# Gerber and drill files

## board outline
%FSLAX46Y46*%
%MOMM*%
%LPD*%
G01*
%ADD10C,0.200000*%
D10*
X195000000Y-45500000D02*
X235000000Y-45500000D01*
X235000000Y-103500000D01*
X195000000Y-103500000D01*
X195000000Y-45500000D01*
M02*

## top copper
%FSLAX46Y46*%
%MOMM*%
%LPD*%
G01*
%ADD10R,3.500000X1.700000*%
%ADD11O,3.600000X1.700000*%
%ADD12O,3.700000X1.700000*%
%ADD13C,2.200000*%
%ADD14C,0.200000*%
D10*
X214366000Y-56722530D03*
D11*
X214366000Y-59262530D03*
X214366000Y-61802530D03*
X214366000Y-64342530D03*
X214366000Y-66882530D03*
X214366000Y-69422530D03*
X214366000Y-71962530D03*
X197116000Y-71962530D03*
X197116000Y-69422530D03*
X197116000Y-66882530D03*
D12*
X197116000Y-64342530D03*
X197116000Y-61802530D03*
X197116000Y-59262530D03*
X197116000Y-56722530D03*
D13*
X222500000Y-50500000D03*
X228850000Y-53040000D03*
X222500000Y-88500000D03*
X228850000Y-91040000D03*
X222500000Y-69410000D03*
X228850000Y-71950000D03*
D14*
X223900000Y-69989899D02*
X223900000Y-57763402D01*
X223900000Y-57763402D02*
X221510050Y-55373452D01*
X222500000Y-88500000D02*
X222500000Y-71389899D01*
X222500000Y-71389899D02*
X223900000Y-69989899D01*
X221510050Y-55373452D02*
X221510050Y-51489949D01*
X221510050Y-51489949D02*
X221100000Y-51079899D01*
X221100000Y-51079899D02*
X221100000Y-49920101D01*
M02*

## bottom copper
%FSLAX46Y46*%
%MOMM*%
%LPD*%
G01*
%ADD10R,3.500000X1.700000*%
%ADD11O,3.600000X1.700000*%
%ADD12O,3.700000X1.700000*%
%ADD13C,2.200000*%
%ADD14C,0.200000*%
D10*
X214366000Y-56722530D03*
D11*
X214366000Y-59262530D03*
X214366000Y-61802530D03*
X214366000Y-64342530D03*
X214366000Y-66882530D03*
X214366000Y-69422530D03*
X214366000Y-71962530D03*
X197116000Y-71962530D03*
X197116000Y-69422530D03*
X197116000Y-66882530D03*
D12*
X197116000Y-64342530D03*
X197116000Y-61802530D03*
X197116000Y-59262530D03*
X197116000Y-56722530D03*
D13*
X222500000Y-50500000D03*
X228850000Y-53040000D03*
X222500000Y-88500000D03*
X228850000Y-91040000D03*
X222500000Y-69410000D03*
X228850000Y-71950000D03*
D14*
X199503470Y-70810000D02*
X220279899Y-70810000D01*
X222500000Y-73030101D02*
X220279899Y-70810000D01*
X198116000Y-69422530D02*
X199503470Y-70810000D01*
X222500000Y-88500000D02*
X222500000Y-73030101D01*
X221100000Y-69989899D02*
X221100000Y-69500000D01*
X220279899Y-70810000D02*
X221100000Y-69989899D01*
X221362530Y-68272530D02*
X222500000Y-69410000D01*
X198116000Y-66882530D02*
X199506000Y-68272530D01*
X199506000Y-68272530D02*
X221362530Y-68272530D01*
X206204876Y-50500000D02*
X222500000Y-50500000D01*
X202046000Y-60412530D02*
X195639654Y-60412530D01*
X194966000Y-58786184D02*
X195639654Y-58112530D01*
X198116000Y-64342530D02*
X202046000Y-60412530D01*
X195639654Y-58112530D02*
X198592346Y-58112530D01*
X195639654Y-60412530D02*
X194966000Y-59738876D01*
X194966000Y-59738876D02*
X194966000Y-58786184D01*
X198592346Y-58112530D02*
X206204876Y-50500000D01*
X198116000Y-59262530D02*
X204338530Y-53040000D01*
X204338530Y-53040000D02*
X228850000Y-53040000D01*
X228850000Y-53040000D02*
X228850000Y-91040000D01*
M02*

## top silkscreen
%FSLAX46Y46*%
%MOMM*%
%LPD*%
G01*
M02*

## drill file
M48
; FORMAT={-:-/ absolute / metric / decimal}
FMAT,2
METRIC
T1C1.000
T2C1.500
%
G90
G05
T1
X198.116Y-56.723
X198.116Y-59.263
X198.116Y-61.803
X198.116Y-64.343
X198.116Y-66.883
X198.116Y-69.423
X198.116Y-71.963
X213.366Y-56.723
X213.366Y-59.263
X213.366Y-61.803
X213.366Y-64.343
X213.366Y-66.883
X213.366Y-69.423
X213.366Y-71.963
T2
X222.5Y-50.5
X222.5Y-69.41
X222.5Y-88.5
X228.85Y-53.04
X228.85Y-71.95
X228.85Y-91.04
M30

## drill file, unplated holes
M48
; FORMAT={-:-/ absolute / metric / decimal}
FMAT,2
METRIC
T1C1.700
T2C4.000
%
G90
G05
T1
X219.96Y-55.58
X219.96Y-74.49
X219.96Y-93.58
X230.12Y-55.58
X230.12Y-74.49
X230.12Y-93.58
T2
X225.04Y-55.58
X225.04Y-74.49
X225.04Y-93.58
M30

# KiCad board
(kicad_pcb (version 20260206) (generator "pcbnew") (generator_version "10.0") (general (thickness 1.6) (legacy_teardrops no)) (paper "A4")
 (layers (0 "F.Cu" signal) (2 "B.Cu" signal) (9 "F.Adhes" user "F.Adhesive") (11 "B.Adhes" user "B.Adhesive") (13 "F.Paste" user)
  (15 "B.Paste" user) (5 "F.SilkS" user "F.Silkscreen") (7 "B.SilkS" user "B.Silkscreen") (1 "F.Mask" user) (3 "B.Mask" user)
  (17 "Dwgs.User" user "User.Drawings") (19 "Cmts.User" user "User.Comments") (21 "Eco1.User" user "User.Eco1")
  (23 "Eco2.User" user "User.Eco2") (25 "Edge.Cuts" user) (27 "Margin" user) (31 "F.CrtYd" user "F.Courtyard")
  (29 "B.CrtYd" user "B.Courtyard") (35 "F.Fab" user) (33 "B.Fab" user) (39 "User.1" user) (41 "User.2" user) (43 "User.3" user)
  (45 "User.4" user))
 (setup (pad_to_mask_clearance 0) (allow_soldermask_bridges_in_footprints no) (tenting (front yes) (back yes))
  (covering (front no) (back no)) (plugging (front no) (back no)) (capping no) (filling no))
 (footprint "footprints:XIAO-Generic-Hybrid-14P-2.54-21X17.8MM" (layer "B.Cu") (at 205.741 64.34253 180)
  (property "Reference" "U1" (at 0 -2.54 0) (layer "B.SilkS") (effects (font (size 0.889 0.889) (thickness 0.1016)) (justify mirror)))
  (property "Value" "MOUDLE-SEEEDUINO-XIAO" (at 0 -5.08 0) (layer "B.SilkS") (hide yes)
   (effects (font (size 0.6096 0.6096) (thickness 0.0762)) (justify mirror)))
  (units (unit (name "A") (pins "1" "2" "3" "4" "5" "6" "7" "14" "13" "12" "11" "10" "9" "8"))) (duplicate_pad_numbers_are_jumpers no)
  (pad "1" thru_hole rect (at -7.625 7.62 180) (size 3.5 1.7) (drill 1 (offset -1 0)) (layers "*.Cu" "*.Mask") (remove_unused_layers no)
   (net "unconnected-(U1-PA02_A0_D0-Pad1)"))
  (pad "2" thru_hole oval (at -7.625 5.08 180) (size 3.6 1.7) (drill 1 (offset -1 0)) (layers "*.Cu" "*.Mask") (remove_unused_layers no)
   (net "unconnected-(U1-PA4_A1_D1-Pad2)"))
  (pad "3" thru_hole oval (at -7.625 2.54 180) (size 3.6 1.7) (drill 1 (offset -1 0)) (layers "*.Cu" "*.Mask") (remove_unused_layers no)
   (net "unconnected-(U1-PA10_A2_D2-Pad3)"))
  (pad "4" thru_hole oval (at -7.625 0 180) (size 3.6 1.7) (drill 1 (offset -1 0)) (layers "*.Cu" "*.Mask") (remove_unused_layers no)
   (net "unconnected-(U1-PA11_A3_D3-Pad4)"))
  (pad "5" thru_hole oval (at -7.625 -2.54 180) (size 3.6 1.7) (drill 1 (offset -1 0)) (layers "*.Cu" "*.Mask") (remove_unused_layers no)
   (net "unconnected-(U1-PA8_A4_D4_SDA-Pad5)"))
  (pad "6" thru_hole oval (at -7.625 -5.08) (size 3.6 1.7) (drill 1 (offset 1 0)) (layers "*.Cu" "*.Mask") (remove_unused_layers no)
   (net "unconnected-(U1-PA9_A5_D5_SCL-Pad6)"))
  (pad "7" thru_hole oval (at -7.625 -7.62 180) (size 3.6 1.7) (drill 1 (offset -1 0)) (layers "*.Cu" "*.Mask") (remove_unused_layers no)
   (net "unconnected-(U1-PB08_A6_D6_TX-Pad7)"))
  (pad "8" thru_hole oval (at 7.625 -7.62 180) (size 3.6 1.7) (drill 1 (offset 1 0)) (layers "*.Cu" "*.Mask") (remove_unused_layers no)
   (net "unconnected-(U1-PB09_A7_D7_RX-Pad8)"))
  (pad "9" thru_hole oval (at 7.625 -5.08 180) (size 3.6 1.7) (drill 1 (offset 1 0)) (layers "*.Cu" "*.Mask") (remove_unused_layers no)
   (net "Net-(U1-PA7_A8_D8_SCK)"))
  (pad "10" thru_hole oval (at 7.625 -2.54 180) (size 3.6 1.7) (drill 1 (offset 1 0)) (layers "*.Cu" "*.Mask") (remove_unused_layers no)
   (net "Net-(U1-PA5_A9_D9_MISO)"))
  (pad "11" thru_hole oval (at 7.625 0 180) (size 3.7 1.7) (drill 1 (offset 1 0)) (layers "*.Cu" "*.Mask") (remove_unused_layers no)
   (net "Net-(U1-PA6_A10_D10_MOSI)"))
  (pad "12" thru_hole oval (at 7.625 2.54 180) (size 3.7 1.7) (drill 1 (offset 1 0)) (layers "*.Cu" "*.Mask") (remove_unused_layers no)
   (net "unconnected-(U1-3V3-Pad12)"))
  (pad "13" thru_hole oval (at 7.625 5.08 180) (size 3.7 1.7) (drill 1 (offset 1 0)) (layers "*.Cu" "*.Mask") (remove_unused_layers no)
   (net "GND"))
  (pad "14" thru_hole oval (at 7.625 7.62 180) (size 3.7 1.7) (drill 1 (offset 1 0)) (layers "*.Cu" "*.Mask") (remove_unused_layers no)
   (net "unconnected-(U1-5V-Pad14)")))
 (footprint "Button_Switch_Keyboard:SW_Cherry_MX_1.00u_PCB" (layer "B.Cu") (at 222.5 50.5 180)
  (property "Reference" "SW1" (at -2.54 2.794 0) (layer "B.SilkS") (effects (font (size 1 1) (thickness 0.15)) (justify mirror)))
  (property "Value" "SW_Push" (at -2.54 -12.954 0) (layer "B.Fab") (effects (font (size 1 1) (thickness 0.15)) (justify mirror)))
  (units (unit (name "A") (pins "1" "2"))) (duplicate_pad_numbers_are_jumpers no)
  (pad "" np_thru_hole circle (at -7.62 -5.08 180) (size 1.7 1.7) (drill 1.7) (layers "*.Cu" "*.Mask"))
  (pad "" np_thru_hole circle (at -2.54 -5.08 180) (size 4 4) (drill 4) (layers "*.Cu" "*.Mask"))
  (pad "" np_thru_hole circle (at 2.54 -5.08 180) (size 1.7 1.7) (drill 1.7) (layers "*.Cu" "*.Mask"))
  (pad "1" thru_hole circle (at 0 0 180) (size 2.2 2.2) (drill 1.5) (layers "*.Cu" "*.Mask") (remove_unused_layers no)
   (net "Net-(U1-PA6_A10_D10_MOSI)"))
  (pad "2" thru_hole circle (at -6.35 -2.54 180) (size 2.2 2.2) (drill 1.5) (layers "*.Cu" "*.Mask") (remove_unused_layers no) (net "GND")))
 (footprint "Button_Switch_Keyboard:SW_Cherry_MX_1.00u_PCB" (layer "B.Cu") (at 222.5 88.5 180)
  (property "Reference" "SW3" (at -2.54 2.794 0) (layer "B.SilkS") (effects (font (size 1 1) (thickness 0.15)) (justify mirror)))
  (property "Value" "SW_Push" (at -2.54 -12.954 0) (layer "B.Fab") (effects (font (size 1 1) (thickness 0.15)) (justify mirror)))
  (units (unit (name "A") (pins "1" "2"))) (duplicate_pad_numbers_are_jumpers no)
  (pad "" np_thru_hole circle (at -7.62 -5.08 180) (size 1.7 1.7) (drill 1.7) (layers "*.Cu" "*.Mask"))
  (pad "" np_thru_hole circle (at -2.54 -5.08 180) (size 4 4) (drill 4) (layers "*.Cu" "*.Mask"))
  (pad "" np_thru_hole circle (at 2.54 -5.08 180) (size 1.7 1.7) (drill 1.7) (layers "*.Cu" "*.Mask"))
  (pad "1" thru_hole circle (at 0 0 180) (size 2.2 2.2) (drill 1.5) (layers "*.Cu" "*.Mask") (remove_unused_layers no)
   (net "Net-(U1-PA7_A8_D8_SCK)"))
  (pad "2" thru_hole circle (at -6.35 -2.54 180) (size 2.2 2.2) (drill 1.5) (layers "*.Cu" "*.Mask") (remove_unused_layers no) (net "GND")))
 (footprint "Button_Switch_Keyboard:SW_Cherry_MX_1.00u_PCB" (layer "B.Cu") (at 222.5 69.41 180)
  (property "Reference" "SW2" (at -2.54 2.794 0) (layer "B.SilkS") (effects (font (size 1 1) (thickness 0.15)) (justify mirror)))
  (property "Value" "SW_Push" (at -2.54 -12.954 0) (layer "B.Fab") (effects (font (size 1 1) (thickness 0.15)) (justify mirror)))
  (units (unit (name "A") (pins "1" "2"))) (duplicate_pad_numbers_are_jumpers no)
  (pad "" np_thru_hole circle (at -7.62 -5.08 180) (size 1.7 1.7) (drill 1.7) (layers "*.Cu" "*.Mask"))
  (pad "" np_thru_hole circle (at -2.54 -5.08 180) (size 4 4) (drill 4) (layers "*.Cu" "*.Mask"))
  (pad "" np_thru_hole circle (at 2.54 -5.08 180) (size 1.7 1.7) (drill 1.7) (layers "*.Cu" "*.Mask"))
  (pad "1" thru_hole circle (at 0 0 180) (size 2.2 2.2) (drill 1.5) (layers "*.Cu" "*.Mask") (remove_unused_layers no)
   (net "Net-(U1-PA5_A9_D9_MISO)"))
  (pad "2" thru_hole circle (at -6.35 -2.54 180) (size 2.2 2.2) (drill 1.5) (layers "*.Cu" "*.Mask") (remove_unused_layers no) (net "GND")))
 (gr_rect (start 195 45.5) (end 235 103.5) (stroke (width 0.2) (type solid)) (fill no) (layer "Edge.Cuts"))
 (segment (start 223.9 69.989899) (end 223.9 57.763402) (width 0.2) (layer "F.Cu") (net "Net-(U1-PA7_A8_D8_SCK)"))
 (segment (start 223.9 57.763402) (end 221.51005 55.373452) (width 0.2) (layer "F.Cu") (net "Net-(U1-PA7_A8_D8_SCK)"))
 (segment (start 222.5 88.5) (end 222.5 71.389899) (width 0.2) (layer "F.Cu") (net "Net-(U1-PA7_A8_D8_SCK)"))
 (segment (start 222.5 71.389899) (end 223.9 69.989899) (width 0.2) (layer "F.Cu") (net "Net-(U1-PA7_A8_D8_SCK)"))
 (segment (start 221.51005 55.373452) (end 221.51005 51.489949) (width 0.2) (layer "F.Cu") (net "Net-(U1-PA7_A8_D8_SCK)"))
 (segment (start 221.51005 51.489949) (end 221.1 51.079899) (width 0.2) (layer "F.Cu") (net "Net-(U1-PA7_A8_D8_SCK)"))
 (segment (start 221.1 51.079899) (end 221.1 49.920101) (width 0.2) (layer "F.Cu") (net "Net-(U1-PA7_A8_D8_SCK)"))
 (segment (start 199.50347 70.81) (end 220.279899 70.81) (width 0.2) (layer "B.Cu") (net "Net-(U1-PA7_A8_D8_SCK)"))
 (segment (start 222.5 73.030101) (end 220.279899 70.81) (width 0.2) (layer "B.Cu") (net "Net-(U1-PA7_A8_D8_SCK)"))
 (segment (start 198.116 69.42253) (end 199.50347 70.81) (width 0.2) (layer "B.Cu") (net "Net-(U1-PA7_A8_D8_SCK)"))
 (segment (start 222.5 88.5) (end 222.5 73.030101) (width 0.2) (layer "B.Cu") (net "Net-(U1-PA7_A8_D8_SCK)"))
 (segment (start 221.1 69.989899) (end 221.1 69.5) (width 0.2) (layer "B.Cu") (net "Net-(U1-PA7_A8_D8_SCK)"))
 (segment (start 220.279899 70.81) (end 221.1 69.989899) (width 0.2) (layer "B.Cu") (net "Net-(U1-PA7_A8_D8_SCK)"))
 (segment (start 221.36253 68.27253) (end 222.5 69.41) (width 0.2) (layer "B.Cu") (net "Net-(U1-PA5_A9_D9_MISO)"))
 (segment (start 198.116 66.88253) (end 199.506 68.27253) (width 0.2) (layer "B.Cu") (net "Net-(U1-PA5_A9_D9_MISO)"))
 (segment (start 199.506 68.27253) (end 221.36253 68.27253) (width 0.2) (layer "B.Cu") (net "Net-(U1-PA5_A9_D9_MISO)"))
 (segment (start 206.204876 50.5) (end 222.5 50.5) (width 0.2) (layer "B.Cu") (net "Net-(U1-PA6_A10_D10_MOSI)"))
 (segment (start 202.046 60.41253) (end 195.639654 60.41253) (width 0.2) (layer "B.Cu") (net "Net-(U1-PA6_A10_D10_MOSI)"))
 (segment (start 194.966 58.786184) (end 195.639654 58.11253) (width 0.2) (layer "B.Cu") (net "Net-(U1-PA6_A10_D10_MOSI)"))
 (segment (start 198.116 64.34253) (end 202.046 60.41253) (width 0.2) (layer "B.Cu") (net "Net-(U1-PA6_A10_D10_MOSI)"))
 (segment (start 195.639654 58.11253) (end 198.592346 58.11253) (width 0.2) (layer "B.Cu") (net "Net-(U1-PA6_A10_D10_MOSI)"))
 (segment (start 195.639654 60.41253) (end 194.966 59.738876) (width 0.2) (layer "B.Cu") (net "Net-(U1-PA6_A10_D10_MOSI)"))
 (segment (start 194.966 59.738876) (end 194.966 58.786184) (width 0.2) (layer "B.Cu") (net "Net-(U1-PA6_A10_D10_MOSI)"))
 (segment (start 198.592346 58.11253) (end 206.204876 50.5) (width 0.2) (layer "B.Cu") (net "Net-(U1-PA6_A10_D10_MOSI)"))
 (segment (start 198.116 59.26253) (end 204.33853 53.04) (width 0.2) (layer "B.Cu") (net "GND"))
 (segment (start 204.33853 53.04) (end 228.85 53.04) (width 0.2) (layer "B.Cu") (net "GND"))
 (segment (start 228.85 53.04) (end 228.85 91.04) (width 0.2) (layer "B.Cu") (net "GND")))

